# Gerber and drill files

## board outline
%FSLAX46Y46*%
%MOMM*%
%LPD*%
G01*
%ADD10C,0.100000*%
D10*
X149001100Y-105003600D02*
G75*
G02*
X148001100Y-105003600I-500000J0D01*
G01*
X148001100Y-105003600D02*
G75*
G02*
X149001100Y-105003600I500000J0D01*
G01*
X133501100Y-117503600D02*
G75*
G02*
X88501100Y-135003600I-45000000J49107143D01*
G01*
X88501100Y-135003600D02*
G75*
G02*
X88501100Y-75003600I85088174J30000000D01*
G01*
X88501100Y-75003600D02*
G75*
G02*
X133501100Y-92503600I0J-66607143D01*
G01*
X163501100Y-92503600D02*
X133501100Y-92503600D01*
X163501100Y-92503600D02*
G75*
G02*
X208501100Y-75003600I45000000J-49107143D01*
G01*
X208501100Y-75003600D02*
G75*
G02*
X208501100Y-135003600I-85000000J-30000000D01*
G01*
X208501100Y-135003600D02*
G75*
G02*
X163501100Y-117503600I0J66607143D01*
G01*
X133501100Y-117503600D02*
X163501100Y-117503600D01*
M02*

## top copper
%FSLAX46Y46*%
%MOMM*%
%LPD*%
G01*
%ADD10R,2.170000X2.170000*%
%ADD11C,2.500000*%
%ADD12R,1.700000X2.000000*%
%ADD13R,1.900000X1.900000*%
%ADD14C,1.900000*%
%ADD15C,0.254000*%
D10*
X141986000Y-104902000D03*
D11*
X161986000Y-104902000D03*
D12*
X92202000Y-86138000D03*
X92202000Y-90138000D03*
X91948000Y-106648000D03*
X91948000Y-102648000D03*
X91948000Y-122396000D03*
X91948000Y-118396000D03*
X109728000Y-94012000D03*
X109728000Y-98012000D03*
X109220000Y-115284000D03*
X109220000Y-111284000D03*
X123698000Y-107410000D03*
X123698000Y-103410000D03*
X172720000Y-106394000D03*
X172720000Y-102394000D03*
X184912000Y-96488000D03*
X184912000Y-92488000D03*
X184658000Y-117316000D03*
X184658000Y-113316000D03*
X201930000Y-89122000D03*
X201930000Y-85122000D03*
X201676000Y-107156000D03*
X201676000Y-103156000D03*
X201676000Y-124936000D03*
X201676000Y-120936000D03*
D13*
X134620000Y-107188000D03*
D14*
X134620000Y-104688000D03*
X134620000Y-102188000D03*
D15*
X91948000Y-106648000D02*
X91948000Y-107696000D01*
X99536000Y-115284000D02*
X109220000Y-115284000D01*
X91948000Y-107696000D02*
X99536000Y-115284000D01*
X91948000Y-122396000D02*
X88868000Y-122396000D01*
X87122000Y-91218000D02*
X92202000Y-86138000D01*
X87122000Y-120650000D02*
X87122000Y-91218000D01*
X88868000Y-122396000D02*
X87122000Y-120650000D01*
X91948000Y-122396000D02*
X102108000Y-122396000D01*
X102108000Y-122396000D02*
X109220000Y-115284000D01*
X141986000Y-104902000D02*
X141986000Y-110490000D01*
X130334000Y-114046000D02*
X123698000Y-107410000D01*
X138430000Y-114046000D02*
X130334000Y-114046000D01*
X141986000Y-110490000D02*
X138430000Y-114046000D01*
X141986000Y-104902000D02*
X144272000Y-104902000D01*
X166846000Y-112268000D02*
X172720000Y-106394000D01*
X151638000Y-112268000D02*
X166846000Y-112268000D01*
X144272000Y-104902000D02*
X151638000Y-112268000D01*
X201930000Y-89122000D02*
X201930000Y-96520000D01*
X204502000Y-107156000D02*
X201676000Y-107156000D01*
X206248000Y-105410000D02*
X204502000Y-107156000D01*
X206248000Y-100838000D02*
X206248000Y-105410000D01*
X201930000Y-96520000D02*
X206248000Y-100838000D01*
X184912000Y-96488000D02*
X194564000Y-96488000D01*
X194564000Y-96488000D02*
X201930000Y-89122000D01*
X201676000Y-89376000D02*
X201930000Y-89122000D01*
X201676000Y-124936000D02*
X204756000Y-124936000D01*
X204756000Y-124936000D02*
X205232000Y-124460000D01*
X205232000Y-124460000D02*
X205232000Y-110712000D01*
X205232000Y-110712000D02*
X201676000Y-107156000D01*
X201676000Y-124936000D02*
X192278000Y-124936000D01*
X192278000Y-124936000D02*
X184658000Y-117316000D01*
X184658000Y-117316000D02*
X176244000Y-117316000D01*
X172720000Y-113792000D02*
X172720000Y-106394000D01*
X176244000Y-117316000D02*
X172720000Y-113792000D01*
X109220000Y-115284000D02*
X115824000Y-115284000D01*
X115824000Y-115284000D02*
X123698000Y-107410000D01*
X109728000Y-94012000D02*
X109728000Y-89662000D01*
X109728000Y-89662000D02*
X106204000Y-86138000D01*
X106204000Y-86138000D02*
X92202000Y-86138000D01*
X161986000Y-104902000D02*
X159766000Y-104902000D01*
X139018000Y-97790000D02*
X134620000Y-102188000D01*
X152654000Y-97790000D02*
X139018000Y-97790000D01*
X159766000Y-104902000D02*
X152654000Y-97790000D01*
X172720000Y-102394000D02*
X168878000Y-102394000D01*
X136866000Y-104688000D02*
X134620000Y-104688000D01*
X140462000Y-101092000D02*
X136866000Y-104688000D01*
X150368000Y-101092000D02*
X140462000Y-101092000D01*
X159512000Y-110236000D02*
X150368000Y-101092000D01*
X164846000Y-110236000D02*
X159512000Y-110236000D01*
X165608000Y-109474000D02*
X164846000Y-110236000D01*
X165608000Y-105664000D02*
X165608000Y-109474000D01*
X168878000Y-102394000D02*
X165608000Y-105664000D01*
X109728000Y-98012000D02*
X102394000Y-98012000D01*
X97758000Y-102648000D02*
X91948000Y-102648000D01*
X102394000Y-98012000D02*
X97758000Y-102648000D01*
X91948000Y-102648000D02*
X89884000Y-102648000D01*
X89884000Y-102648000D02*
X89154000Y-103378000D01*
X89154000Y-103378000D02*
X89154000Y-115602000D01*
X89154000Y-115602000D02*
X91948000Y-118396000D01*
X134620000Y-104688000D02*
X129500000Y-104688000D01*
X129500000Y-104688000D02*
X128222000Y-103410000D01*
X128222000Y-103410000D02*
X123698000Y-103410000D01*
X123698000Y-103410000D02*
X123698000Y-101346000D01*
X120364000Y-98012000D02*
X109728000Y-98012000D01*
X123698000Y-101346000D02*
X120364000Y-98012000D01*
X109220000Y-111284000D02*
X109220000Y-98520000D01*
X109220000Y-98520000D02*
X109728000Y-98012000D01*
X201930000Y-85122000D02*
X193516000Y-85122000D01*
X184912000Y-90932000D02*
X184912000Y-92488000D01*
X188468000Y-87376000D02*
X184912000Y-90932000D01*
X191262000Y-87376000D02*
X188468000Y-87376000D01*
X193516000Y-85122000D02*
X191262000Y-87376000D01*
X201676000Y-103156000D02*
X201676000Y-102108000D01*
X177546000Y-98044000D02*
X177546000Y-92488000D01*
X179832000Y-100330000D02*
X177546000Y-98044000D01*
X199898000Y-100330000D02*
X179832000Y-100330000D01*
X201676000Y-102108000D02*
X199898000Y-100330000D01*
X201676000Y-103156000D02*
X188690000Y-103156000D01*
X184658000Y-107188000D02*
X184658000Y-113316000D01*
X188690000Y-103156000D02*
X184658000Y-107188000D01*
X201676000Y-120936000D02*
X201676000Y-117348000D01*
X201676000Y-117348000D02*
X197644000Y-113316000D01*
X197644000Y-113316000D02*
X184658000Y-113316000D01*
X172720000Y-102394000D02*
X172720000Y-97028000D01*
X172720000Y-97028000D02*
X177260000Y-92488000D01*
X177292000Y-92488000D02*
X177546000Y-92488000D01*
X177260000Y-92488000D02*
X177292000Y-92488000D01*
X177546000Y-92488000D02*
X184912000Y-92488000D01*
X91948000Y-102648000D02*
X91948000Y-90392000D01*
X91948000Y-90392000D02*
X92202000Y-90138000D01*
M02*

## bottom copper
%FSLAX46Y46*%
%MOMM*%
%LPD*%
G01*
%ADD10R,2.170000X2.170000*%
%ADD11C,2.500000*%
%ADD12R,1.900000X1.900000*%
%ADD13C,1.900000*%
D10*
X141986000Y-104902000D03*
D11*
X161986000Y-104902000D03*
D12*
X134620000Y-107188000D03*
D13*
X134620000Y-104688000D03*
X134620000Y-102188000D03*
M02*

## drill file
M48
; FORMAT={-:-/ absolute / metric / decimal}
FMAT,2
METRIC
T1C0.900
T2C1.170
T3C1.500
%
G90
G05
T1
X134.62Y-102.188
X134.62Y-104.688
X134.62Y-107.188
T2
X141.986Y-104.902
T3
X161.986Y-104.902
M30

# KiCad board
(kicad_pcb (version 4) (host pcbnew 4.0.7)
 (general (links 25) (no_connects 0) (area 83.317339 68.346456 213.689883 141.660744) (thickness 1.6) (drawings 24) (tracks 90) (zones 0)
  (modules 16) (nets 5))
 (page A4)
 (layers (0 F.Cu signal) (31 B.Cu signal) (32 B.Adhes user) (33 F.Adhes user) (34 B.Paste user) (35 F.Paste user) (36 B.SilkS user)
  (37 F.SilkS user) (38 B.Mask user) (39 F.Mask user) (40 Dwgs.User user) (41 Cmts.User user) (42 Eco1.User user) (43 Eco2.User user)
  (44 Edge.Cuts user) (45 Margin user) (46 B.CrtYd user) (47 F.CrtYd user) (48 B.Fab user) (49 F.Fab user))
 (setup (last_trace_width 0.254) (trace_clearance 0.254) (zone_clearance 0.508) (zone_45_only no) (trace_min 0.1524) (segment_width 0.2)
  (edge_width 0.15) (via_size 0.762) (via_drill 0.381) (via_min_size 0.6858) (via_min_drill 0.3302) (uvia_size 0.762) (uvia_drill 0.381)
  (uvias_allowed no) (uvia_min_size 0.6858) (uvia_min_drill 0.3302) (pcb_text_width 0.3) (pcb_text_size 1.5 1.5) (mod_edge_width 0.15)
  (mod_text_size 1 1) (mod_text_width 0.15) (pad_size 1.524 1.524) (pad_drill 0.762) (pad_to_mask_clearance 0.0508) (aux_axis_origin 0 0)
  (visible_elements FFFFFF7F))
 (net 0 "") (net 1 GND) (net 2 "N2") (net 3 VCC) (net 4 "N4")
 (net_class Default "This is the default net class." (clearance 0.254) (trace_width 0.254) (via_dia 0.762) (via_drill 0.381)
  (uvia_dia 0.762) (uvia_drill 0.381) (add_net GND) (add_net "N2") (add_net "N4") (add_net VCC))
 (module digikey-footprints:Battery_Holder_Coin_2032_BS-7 (layer F.Cu) (at 141.986 104.902)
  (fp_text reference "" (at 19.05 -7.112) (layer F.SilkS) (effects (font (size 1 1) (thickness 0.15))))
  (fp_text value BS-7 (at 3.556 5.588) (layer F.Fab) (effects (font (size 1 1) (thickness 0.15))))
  (pad Neg thru_hole rect (at 0 0) (size 2.17 2.17) (drill 1.17) (layers *.Cu *.Mask) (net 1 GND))
  (pad Pos thru_hole circle (at 20 0) (size 2.5 2.5) (drill 1.5) (layers *.Cu *.Mask) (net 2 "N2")))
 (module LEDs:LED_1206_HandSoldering (layer F.Cu) (at 92.202 88.138 270)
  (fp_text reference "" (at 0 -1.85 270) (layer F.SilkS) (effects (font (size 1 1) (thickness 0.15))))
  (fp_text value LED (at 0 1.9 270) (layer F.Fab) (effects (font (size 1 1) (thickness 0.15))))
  (pad 1 smd rect (at -2 0 270) (size 2 1.7) (layers F.Cu F.Paste F.Mask) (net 1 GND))
  (pad 2 smd rect (at 2 0 270) (size 2 1.7) (layers F.Cu F.Paste F.Mask) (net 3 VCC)))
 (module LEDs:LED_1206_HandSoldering (layer F.Cu) (at 91.948 104.648 90)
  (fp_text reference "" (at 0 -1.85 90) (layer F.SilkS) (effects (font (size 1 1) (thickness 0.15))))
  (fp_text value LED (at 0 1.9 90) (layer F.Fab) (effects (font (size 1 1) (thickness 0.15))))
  (pad 1 smd rect (at -2 0 90) (size 2 1.7) (layers F.Cu F.Paste F.Mask) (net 1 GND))
  (pad 2 smd rect (at 2 0 90) (size 2 1.7) (layers F.Cu F.Paste F.Mask) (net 3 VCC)))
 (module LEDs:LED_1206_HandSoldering (layer F.Cu) (at 91.948 120.396 90)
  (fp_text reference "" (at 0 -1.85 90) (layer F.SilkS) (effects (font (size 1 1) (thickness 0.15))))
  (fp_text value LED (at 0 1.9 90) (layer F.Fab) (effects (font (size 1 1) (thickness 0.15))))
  (pad 1 smd rect (at -2 0 90) (size 2 1.7) (layers F.Cu F.Paste F.Mask) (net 1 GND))
  (pad 2 smd rect (at 2 0 90) (size 2 1.7) (layers F.Cu F.Paste F.Mask) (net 3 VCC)))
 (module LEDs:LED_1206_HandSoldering (layer F.Cu) (at 109.728 96.012 270)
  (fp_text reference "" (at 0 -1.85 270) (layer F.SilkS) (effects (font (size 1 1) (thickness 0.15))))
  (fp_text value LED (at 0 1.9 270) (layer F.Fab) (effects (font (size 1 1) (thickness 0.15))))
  (pad 1 smd rect (at -2 0 270) (size 2 1.7) (layers F.Cu F.Paste F.Mask) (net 1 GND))
  (pad 2 smd rect (at 2 0 270) (size 2 1.7) (layers F.Cu F.Paste F.Mask) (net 3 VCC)))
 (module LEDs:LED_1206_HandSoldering (layer F.Cu) (at 109.22 113.284 90)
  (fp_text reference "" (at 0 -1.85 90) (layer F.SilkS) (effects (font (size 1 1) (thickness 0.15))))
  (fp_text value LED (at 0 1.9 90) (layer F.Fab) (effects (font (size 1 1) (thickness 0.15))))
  (pad 1 smd rect (at -2 0 90) (size 2 1.7) (layers F.Cu F.Paste F.Mask) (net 1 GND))
  (pad 2 smd rect (at 2 0 90) (size 2 1.7) (layers F.Cu F.Paste F.Mask) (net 3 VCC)))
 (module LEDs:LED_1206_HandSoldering (layer F.Cu) (at 123.698 105.41 90)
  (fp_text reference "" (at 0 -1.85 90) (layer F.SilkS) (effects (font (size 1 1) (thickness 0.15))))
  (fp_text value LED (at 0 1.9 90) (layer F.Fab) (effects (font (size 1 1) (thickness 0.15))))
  (pad 1 smd rect (at -2 0 90) (size 2 1.7) (layers F.Cu F.Paste F.Mask) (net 1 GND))
  (pad 2 smd rect (at 2 0 90) (size 2 1.7) (layers F.Cu F.Paste F.Mask) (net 3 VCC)))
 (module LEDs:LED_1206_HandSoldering (layer F.Cu) (at 172.72 104.394 90)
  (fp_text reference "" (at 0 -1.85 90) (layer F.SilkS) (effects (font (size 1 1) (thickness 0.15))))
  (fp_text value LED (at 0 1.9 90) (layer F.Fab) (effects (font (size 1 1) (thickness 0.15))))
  (pad 1 smd rect (at -2 0 90) (size 2 1.7) (layers F.Cu F.Paste F.Mask) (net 1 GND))
  (pad 2 smd rect (at 2 0 90) (size 2 1.7) (layers F.Cu F.Paste F.Mask) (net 3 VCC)))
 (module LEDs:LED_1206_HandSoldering (layer F.Cu) (at 184.912 94.488 90)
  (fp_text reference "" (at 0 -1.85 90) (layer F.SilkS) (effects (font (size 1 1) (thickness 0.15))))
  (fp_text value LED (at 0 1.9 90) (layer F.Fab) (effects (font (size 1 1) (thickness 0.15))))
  (pad 1 smd rect (at -2 0 90) (size 2 1.7) (layers F.Cu F.Paste F.Mask) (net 1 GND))
  (pad 2 smd rect (at 2 0 90) (size 2 1.7) (layers F.Cu F.Paste F.Mask) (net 3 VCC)))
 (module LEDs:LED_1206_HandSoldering (layer F.Cu) (at 184.658 115.316 90)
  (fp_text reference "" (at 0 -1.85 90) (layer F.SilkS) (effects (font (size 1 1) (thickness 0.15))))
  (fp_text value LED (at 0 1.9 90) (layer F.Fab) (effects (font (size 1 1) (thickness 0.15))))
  (pad 1 smd rect (at -2 0 90) (size 2 1.7) (layers F.Cu F.Paste F.Mask) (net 1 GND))
  (pad 2 smd rect (at 2 0 90) (size 2 1.7) (layers F.Cu F.Paste F.Mask) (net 3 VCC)))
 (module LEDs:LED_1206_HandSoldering (layer F.Cu) (at 201.93 87.122 90)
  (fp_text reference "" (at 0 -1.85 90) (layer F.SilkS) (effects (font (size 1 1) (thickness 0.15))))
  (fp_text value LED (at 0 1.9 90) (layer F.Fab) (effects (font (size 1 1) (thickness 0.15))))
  (pad 1 smd rect (at -2 0 90) (size 2 1.7) (layers F.Cu F.Paste F.Mask) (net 1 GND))
  (pad 2 smd rect (at 2 0 90) (size 2 1.7) (layers F.Cu F.Paste F.Mask) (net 3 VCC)))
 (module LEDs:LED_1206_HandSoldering (layer F.Cu) (at 201.676 105.156 90)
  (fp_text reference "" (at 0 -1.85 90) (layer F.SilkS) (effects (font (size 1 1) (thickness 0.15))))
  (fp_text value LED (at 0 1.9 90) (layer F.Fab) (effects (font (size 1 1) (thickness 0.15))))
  (pad 1 smd rect (at -2 0 90) (size 2 1.7) (layers F.Cu F.Paste F.Mask) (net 1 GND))
  (pad 2 smd rect (at 2 0 90) (size 2 1.7) (layers F.Cu F.Paste F.Mask) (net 3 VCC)))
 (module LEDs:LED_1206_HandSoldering (layer F.Cu) (at 201.676 122.936 90)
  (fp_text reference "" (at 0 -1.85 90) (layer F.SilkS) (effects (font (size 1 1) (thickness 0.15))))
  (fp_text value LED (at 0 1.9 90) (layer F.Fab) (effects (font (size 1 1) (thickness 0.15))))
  (pad 1 smd rect (at -2 0 90) (size 2 1.7) (layers F.Cu F.Paste F.Mask) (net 1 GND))
  (pad 2 smd rect (at 2 0 90) (size 2 1.7) (layers F.Cu F.Paste F.Mask) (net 3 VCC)))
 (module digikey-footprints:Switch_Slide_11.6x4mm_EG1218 (layer F.Cu) (at 134.62 107.188 90)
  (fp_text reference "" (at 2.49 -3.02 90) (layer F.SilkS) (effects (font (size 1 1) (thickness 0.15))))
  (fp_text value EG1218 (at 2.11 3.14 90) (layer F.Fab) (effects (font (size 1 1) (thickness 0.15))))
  (pad 1 thru_hole rect (at 0 0 90) (size 1.9 1.9) (drill 0.9) (layers *.Cu *.Mask) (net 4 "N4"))
  (pad 2 thru_hole circle (at 2.5 0 90) (size 1.9 1.9) (drill 0.9) (layers *.Cu *.Mask) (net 3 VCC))
  (pad 3 thru_hole circle (at 5 0 90) (size 1.9 1.9) (drill 0.9) (layers *.Cu *.Mask) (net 2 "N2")))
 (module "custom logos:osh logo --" (layer B.Cu) (at 157.48 96.52 180)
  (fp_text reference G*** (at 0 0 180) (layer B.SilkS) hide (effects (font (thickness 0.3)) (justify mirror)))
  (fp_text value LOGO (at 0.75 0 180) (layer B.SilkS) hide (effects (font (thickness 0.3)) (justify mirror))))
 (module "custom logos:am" (layer B.Cu) (at 141.224 97.028 180)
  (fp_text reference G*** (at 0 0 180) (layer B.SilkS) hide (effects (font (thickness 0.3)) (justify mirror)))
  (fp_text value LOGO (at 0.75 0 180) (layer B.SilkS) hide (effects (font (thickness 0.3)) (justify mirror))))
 (gr_circle (center 148.5011 105.0036) (end 149.0011 105.0036) (layer Edge.Cuts) (width 0.1))
 (gr_arc (start 88.5011 68.396457) (end 88.5011 135.0036) (angle -42.50101101) (layer Edge.Cuts) (width 0.1))
 (gr_arc (start 173.589274 105.0036) (end 88.5011 75.0036) (angle -38.84279692) (layer Edge.Cuts) (width 0.1))
 (gr_arc (start 88.5011 141.610743) (end 133.5011 92.5036) (angle -42.50101101) (layer Edge.Cuts) (width 0.1))
 (gr_line (start 163.5011 92.5036) (end 133.5011 92.5036) (layer Edge.Cuts) (width 0.1))
 (gr_arc (start 208.5011 141.610743) (end 208.5011 75.0036) (angle -42.50101101) (layer Edge.Cuts) (width 0.1))
 (gr_arc (start 123.5011 105.0036) (end 208.5011 135.0036) (angle -38.88006966) (layer Edge.Cuts) (width 0.1))
 (gr_arc (start 208.5011 68.396457) (end 163.5011 117.5036) (angle -42.50101101) (layer Edge.Cuts) (width 0.1))
 (gr_line (start 133.5011 117.5036) (end 163.5011 117.5036) (layer Edge.Cuts) (width 0.1))
 (segment (start 91.948 106.648) (end 91.948 107.696) (width 0.254) (layer F.Cu) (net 1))
 (segment (start 99.536 115.284) (end 109.22 115.284) (width 0.254) (layer F.Cu) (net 1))
 (segment (start 91.948 107.696) (end 99.536 115.284) (width 0.254) (layer F.Cu) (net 1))
 (segment (start 91.948 122.396) (end 88.868 122.396) (width 0.254) (layer F.Cu) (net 1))
 (segment (start 87.122 91.218) (end 92.202 86.138) (width 0.254) (layer F.Cu) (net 1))
 (segment (start 87.122 120.65) (end 87.122 91.218) (width 0.254) (layer F.Cu) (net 1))
 (segment (start 88.868 122.396) (end 87.122 120.65) (width 0.254) (layer F.Cu) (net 1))
 (segment (start 91.948 122.396) (end 102.108 122.396) (width 0.254) (layer F.Cu) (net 1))
 (segment (start 102.108 122.396) (end 109.22 115.284) (width 0.254) (layer F.Cu) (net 1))
 (segment (start 141.986 104.902) (end 141.986 110.49) (width 0.254) (layer F.Cu) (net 1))
 (segment (start 130.334 114.046) (end 123.698 107.41) (width 0.254) (layer F.Cu) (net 1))
 (segment (start 138.43 114.046) (end 130.334 114.046) (width 0.254) (layer F.Cu) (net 1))
 (segment (start 141.986 110.49) (end 138.43 114.046) (width 0.254) (layer F.Cu) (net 1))
 (segment (start 141.986 104.902) (end 144.272 104.902) (width 0.254) (layer F.Cu) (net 1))
 (segment (start 166.846 112.268) (end 172.72 106.394) (width 0.254) (layer F.Cu) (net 1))
 (segment (start 151.638 112.268) (end 166.846 112.268) (width 0.254) (layer F.Cu) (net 1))
 (segment (start 144.272 104.902) (end 151.638 112.268) (width 0.254) (layer F.Cu) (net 1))
 (segment (start 201.93 89.122) (end 201.93 96.52) (width 0.254) (layer F.Cu) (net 1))
 (segment (start 204.502 107.156) (end 201.676 107.156) (width 0.254) (layer F.Cu) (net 1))
 (segment (start 206.248 105.41) (end 204.502 107.156) (width 0.254) (layer F.Cu) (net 1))
 (segment (start 206.248 100.838) (end 206.248 105.41) (width 0.254) (layer F.Cu) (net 1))
 (segment (start 201.93 96.52) (end 206.248 100.838) (width 0.254) (layer F.Cu) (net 1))
 (segment (start 184.912 96.488) (end 194.564 96.488) (width 0.254) (layer F.Cu) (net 1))
 (segment (start 194.564 96.488) (end 201.93 89.122) (width 0.254) (layer F.Cu) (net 1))
 (segment (start 201.676 89.376) (end 201.93 89.122) (width 0.254) (layer F.Cu) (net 1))
 (segment (start 201.676 124.936) (end 204.756 124.936) (width 0.254) (layer F.Cu) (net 1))
 (segment (start 204.756 124.936) (end 205.232 124.46) (width 0.254) (layer F.Cu) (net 1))
 (segment (start 205.232 124.46) (end 205.232 110.712) (width 0.254) (layer F.Cu) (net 1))
 (segment (start 205.232 110.712) (end 201.676 107.156) (width 0.254) (layer F.Cu) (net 1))
 (segment (start 201.676 124.936) (end 192.278 124.936) (width 0.254) (layer F.Cu) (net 1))
 (segment (start 192.278 124.936) (end 184.658 117.316) (width 0.254) (layer F.Cu) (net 1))
 (segment (start 184.658 117.316) (end 176.244 117.316) (width 0.254) (layer F.Cu) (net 1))
 (segment (start 172.72 113.792) (end 172.72 106.394) (width 0.254) (layer F.Cu) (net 1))
 (segment (start 176.244 117.316) (end 172.72 113.792) (width 0.254) (layer F.Cu) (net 1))
 (segment (start 109.22 115.284) (end 115.824 115.284) (width 0.254) (layer F.Cu) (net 1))
 (segment (start 115.824 115.284) (end 123.698 107.41) (width 0.254) (layer F.Cu) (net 1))
 (segment (start 109.728 94.012) (end 109.728 89.662) (width 0.254) (layer F.Cu) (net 1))
 (segment (start 109.728 89.662) (end 106.204 86.138) (width 0.254) (layer F.Cu) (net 1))
 (segment (start 106.204 86.138) (end 92.202 86.138) (width 0.254) (layer F.Cu) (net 1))
 (segment (start 161.986 104.902) (end 159.766 104.902) (width 0.254) (layer F.Cu) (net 2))
 (segment (start 139.018 97.79) (end 134.62 102.188) (width 0.254) (layer F.Cu) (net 2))
 (segment (start 152.654 97.79) (end 139.018 97.79) (width 0.254) (layer F.Cu) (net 2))
 (segment (start 159.766 104.902) (end 152.654 97.79) (width 0.254) (layer F.Cu) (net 2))
 (segment (start 172.72 102.394) (end 168.878 102.394) (width 0.254) (layer F.Cu) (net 3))
 (segment (start 136.866 104.688) (end 134.62 104.688) (width 0.254) (layer F.Cu) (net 3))
 (segment (start 140.462 101.092) (end 136.866 104.688) (width 0.254) (layer F.Cu) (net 3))
 (segment (start 150.368 101.092) (end 140.462 101.092) (width 0.254) (layer F.Cu) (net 3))
 (segment (start 159.512 110.236) (end 150.368 101.092) (width 0.254) (layer F.Cu) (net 3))
 (segment (start 164.846 110.236) (end 159.512 110.236) (width 0.254) (layer F.Cu) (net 3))
 (segment (start 165.608 109.474) (end 164.846 110.236) (width 0.254) (layer F.Cu) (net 3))
 (segment (start 165.608 105.664) (end 165.608 109.474) (width 0.254) (layer F.Cu) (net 3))
 (segment (start 168.878 102.394) (end 165.608 105.664) (width 0.254) (layer F.Cu) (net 3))
 (segment (start 109.728 98.012) (end 102.394 98.012) (width 0.254) (layer F.Cu) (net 3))
 (segment (start 97.758 102.648) (end 91.948 102.648) (width 0.254) (layer F.Cu) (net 3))
 (segment (start 102.394 98.012) (end 97.758 102.648) (width 0.254) (layer F.Cu) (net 3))
 (segment (start 91.948 102.648) (end 89.884 102.648) (width 0.254) (layer F.Cu) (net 3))
 (segment (start 89.884 102.648) (end 89.154 103.378) (width 0.254) (layer F.Cu) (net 3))
 (segment (start 89.154 103.378) (end 89.154 115.602) (width 0.254) (layer F.Cu) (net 3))
 (segment (start 89.154 115.602) (end 91.948 118.396) (width 0.254) (layer F.Cu) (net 3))
 (segment (start 134.62 104.688) (end 129.5 104.688) (width 0.254) (layer F.Cu) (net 3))
 (segment (start 129.5 104.688) (end 128.222 103.41) (width 0.254) (layer F.Cu) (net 3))
 (segment (start 128.222 103.41) (end 123.698 103.41) (width 0.254) (layer F.Cu) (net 3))
 (segment (start 123.698 103.41) (end 123.698 101.346) (width 0.254) (layer F.Cu) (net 3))
 (segment (start 120.364 98.012) (end 109.728 98.012) (width 0.254) (layer F.Cu) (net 3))
 (segment (start 123.698 101.346) (end 120.364 98.012) (width 0.254) (layer F.Cu) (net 3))
 (segment (start 109.22 111.284) (end 109.22 98.52) (width 0.254) (layer F.Cu) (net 3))
 (segment (start 109.22 98.52) (end 109.728 98.012) (width 0.254) (layer F.Cu) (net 3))
 (segment (start 201.93 85.122) (end 193.516 85.122) (width 0.254) (layer F.Cu) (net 3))
 (segment (start 184.912 90.932) (end 184.912 92.488) (width 0.254) (layer F.Cu) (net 3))
 (segment (start 188.468 87.376) (end 184.912 90.932) (width 0.254) (layer F.Cu) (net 3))
 (segment (start 191.262 87.376) (end 188.468 87.376) (width 0.254) (layer F.Cu) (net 3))
 (segment (start 193.516 85.122) (end 191.262 87.376) (width 0.254) (layer F.Cu) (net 3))
 (segment (start 201.676 103.156) (end 201.676 102.108) (width 0.254) (layer F.Cu) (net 3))
 (segment (start 177.546 98.044) (end 177.546 92.488) (width 0.254) (layer F.Cu) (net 3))
 (segment (start 179.832 100.33) (end 177.546 98.044) (width 0.254) (layer F.Cu) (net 3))
 (segment (start 199.898 100.33) (end 179.832 100.33) (width 0.254) (layer F.Cu) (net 3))
 (segment (start 201.676 102.108) (end 199.898 100.33) (width 0.254) (layer F.Cu) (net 3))
 (segment (start 201.676 103.156) (end 188.69 103.156) (width 0.254) (layer F.Cu) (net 3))
 (segment (start 184.658 107.188) (end 184.658 113.316) (width 0.254) (layer F.Cu) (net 3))
 (segment (start 188.69 103.156) (end 184.658 107.188) (width 0.254) (layer F.Cu) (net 3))
 (segment (start 201.676 120.936) (end 201.676 117.348) (width 0.254) (layer F.Cu) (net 3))
 (segment (start 201.676 117.348) (end 197.644 113.316) (width 0.254) (layer F.Cu) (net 3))
 (segment (start 197.644 113.316) (end 184.658 113.316) (width 0.254) (layer F.Cu) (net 3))
 (segment (start 172.72 102.394) (end 172.72 97.028) (width 0.254) (layer F.Cu) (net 3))
 (segment (start 172.72 97.028) (end 177.26 92.488) (width 0.254) (layer F.Cu) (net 3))
 (segment (start 177.292 92.488) (end 177.546 92.488) (width 0.254) (layer F.Cu) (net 3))
 (segment (start 177.26 92.488) (end 177.292 92.488) (width 0.254) (layer F.Cu) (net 3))
 (segment (start 177.546 92.488) (end 184.912 92.488) (width 0.254) (layer F.Cu) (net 3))
 (segment (start 91.948 102.648) (end 91.948 90.392) (width 0.254) (layer F.Cu) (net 3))
 (segment (start 91.948 90.392) (end 92.202 90.138) (width 0.254) (layer F.Cu) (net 3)))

